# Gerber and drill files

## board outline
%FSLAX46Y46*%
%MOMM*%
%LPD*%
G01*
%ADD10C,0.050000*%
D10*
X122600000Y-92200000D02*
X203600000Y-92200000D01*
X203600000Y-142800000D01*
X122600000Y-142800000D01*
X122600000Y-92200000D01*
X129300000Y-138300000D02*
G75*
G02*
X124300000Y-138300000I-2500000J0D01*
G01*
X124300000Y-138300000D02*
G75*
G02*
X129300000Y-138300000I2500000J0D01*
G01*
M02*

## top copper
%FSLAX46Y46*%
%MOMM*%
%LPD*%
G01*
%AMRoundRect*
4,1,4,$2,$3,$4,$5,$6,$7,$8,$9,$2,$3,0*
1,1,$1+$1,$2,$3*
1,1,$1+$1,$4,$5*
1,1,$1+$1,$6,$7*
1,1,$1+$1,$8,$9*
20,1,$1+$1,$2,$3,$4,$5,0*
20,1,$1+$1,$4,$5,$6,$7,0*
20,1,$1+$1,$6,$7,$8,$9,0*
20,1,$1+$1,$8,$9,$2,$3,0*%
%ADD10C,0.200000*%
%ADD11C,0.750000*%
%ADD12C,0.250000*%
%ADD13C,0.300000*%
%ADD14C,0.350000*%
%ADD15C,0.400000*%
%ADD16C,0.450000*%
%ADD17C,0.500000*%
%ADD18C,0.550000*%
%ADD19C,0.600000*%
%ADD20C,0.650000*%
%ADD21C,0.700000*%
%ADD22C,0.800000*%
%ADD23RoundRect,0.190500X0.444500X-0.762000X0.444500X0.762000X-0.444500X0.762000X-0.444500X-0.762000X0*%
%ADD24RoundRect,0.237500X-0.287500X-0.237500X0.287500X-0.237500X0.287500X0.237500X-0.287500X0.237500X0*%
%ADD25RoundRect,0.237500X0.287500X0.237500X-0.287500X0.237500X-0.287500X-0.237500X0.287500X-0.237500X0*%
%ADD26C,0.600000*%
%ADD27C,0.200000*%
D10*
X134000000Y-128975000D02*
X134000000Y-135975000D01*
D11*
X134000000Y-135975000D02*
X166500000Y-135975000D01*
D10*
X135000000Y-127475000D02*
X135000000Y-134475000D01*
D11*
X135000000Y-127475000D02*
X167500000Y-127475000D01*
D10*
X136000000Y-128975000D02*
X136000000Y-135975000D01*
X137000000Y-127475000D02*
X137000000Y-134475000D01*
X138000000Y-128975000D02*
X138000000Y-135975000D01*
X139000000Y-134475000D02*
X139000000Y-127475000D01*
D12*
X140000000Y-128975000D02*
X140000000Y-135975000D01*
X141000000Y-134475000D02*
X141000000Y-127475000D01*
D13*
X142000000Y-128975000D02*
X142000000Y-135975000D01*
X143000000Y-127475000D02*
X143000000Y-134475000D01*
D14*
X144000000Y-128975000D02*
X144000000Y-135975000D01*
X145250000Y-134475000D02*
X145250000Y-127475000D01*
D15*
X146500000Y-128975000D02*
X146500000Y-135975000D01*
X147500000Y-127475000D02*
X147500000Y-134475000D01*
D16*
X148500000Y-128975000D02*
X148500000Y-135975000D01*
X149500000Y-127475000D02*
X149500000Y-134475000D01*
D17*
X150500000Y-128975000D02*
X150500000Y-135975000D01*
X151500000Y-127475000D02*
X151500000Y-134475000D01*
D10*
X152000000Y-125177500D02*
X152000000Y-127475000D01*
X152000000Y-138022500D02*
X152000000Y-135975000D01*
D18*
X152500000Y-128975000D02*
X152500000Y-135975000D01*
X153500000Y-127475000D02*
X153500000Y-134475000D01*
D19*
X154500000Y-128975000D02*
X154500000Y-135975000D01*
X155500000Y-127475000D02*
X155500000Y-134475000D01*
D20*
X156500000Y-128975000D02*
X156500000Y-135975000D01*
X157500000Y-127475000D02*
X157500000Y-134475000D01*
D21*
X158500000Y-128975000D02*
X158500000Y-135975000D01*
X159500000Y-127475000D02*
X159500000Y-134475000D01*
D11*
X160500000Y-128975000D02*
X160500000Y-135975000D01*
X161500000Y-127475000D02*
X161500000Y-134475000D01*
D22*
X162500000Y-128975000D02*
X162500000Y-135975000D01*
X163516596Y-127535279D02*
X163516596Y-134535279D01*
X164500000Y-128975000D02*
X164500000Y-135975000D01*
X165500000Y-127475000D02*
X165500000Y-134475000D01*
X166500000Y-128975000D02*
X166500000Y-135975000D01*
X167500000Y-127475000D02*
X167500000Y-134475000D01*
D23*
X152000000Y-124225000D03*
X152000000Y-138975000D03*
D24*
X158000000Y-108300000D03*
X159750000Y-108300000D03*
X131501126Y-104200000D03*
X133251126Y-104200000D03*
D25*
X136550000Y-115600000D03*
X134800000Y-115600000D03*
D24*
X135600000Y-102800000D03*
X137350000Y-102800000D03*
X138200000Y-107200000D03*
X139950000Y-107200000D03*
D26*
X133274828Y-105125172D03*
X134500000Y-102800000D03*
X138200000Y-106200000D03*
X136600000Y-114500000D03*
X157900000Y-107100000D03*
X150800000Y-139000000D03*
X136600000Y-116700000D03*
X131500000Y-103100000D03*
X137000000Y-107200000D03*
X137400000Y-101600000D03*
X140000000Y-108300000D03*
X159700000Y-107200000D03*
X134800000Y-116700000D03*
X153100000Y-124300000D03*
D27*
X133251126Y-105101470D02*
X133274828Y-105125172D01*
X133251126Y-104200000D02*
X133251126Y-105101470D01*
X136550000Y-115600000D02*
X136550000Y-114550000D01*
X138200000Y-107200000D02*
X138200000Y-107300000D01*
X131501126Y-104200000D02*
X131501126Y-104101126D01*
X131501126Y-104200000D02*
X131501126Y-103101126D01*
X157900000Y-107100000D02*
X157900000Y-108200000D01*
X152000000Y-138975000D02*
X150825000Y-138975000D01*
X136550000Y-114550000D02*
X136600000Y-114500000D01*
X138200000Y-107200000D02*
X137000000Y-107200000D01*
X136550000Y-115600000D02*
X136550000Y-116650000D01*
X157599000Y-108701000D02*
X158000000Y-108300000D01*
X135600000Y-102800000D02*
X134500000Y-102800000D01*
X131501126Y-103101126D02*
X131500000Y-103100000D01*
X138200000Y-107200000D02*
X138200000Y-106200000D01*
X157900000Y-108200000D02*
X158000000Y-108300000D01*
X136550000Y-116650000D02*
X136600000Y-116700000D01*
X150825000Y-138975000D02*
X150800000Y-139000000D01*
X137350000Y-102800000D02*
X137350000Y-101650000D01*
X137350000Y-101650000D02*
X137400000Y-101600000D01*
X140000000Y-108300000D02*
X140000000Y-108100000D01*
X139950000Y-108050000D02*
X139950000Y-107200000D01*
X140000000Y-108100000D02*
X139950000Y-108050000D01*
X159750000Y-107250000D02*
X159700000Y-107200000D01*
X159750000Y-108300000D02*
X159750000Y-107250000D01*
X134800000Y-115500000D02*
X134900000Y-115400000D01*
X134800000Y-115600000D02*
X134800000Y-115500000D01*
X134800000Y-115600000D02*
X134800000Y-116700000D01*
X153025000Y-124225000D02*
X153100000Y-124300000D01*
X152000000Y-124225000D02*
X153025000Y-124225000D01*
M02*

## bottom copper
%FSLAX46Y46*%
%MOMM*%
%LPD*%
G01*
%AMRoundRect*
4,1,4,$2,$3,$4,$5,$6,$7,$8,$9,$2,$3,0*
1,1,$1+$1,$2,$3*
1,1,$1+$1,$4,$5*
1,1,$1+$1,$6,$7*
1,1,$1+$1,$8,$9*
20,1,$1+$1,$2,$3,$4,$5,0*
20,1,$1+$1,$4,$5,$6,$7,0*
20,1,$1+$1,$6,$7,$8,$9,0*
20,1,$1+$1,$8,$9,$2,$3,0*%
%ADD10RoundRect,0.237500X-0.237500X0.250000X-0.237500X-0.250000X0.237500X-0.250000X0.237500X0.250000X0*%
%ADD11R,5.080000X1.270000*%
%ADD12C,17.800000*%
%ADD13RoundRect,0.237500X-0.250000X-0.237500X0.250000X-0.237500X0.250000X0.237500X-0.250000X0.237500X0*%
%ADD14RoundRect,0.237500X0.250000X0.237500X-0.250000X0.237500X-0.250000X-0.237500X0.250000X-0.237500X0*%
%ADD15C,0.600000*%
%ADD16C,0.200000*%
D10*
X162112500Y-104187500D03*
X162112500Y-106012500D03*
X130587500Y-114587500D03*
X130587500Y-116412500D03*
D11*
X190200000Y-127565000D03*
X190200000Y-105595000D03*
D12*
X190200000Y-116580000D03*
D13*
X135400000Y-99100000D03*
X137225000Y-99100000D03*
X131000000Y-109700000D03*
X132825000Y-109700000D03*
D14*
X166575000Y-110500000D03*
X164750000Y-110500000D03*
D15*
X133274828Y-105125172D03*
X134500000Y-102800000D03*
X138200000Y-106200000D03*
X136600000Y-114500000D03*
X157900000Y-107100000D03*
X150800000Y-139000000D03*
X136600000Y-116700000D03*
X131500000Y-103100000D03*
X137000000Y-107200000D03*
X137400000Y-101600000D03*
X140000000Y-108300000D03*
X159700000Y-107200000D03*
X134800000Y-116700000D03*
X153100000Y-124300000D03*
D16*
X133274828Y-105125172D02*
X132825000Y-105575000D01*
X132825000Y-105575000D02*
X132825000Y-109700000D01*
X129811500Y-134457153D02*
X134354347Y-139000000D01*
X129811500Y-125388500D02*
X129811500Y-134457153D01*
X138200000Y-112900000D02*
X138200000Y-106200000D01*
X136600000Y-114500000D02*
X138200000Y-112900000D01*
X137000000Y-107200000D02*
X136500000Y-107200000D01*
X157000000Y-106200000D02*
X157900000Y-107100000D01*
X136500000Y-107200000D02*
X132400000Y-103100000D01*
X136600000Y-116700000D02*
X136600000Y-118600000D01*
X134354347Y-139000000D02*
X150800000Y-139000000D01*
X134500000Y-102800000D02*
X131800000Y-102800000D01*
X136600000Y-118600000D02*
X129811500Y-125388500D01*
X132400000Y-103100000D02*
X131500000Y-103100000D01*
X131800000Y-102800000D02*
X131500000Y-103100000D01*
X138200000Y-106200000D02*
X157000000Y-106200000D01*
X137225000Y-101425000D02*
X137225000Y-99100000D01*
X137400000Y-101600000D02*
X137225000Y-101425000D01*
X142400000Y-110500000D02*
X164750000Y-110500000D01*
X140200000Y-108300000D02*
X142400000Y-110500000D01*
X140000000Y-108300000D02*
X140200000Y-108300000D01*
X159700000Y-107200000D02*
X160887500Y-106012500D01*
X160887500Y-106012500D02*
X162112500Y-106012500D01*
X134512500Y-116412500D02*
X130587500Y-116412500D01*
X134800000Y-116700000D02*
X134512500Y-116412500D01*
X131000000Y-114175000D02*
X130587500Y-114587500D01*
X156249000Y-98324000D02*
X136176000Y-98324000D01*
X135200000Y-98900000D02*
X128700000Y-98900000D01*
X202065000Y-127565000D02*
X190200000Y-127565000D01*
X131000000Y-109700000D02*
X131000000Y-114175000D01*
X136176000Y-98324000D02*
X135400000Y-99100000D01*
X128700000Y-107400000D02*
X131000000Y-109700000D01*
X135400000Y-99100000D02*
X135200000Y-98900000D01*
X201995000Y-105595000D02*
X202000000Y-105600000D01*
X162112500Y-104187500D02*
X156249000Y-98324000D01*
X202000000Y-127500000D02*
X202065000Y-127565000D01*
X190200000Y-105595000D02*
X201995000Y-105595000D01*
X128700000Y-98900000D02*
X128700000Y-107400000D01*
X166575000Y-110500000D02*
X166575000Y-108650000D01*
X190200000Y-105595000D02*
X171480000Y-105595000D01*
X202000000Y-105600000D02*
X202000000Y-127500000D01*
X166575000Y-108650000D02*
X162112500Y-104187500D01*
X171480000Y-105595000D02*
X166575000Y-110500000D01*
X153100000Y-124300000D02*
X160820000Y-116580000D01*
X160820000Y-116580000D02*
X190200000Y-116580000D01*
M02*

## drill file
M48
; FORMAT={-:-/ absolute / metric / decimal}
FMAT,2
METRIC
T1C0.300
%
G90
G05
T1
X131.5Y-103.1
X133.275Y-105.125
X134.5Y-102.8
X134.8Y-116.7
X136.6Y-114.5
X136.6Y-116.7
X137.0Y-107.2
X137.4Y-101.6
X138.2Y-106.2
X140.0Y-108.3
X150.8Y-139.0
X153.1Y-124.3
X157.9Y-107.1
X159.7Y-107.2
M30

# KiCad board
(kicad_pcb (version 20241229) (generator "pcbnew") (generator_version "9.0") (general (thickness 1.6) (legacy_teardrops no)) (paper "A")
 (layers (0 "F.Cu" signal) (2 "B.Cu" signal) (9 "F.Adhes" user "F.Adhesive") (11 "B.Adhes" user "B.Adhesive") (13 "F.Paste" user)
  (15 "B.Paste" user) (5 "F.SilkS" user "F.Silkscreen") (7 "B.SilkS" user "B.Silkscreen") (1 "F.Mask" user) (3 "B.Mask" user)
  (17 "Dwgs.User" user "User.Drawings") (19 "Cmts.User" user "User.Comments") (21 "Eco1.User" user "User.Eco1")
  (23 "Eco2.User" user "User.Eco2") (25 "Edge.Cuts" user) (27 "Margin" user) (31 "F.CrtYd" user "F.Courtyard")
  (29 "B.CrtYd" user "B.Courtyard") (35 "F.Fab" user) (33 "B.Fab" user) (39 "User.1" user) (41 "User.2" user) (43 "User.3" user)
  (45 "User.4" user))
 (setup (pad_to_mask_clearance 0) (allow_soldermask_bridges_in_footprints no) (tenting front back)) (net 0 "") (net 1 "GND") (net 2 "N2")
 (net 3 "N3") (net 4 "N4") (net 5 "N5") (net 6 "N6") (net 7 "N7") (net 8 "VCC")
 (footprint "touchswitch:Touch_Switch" (layer "F.Cu") (at 152 131.475 90)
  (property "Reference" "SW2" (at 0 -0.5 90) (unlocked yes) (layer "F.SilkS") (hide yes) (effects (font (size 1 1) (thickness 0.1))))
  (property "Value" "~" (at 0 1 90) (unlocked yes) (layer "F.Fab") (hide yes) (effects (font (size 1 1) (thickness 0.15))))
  (fp_line (start 2.5 -18) (end -4.5 -18) (stroke (width 0.2) (type default)) (layer "F.Cu"))
  (fp_line (start -4.5 -18) (end -4.5 14.5) (stroke (width 0.75) (type default)) (layer "F.Cu"))
  (fp_line (start 4 -17) (end -3 -17) (stroke (width 0.2) (type default)) (layer "F.Cu"))
  (fp_line (start 4 -17) (end 4 15.5) (stroke (width 0.75) (type default)) (layer "F.Cu"))
  (fp_line (start 2.5 -16) (end -4.5 -16) (stroke (width 0.2) (type default)) (layer "F.Cu"))
  (fp_line (start 4 -15) (end -3 -15) (stroke (width 0.2) (type default)) (layer "F.Cu"))
  (fp_line (start 2.5 -14) (end -4.5 -14) (stroke (width 0.2) (type default)) (layer "F.Cu"))
  (fp_line (start -3 -13) (end 4 -13) (stroke (width 0.2) (type default)) (layer "F.Cu"))
  (fp_line (start 2.5 -12) (end -4.5 -12) (stroke (width 0.25) (type default)) (layer "F.Cu"))
  (fp_line (start -3 -11) (end 4 -11) (stroke (width 0.25) (type default)) (layer "F.Cu"))
  (fp_line (start 2.5 -10) (end -4.5 -10) (stroke (width 0.3) (type default)) (layer "F.Cu"))
  (fp_line (start 4 -9) (end -3 -9) (stroke (width 0.3) (type default)) (layer "F.Cu"))
  (fp_line (start 2.5 -8) (end -4.5 -8) (stroke (width 0.35) (type default)) (layer "F.Cu"))
  (fp_line (start -3 -6.75) (end 4 -6.75) (stroke (width 0.35) (type default)) (layer "F.Cu"))
  (fp_line (start 2.5 -5.5) (end -4.5 -5.5) (stroke (width 0.4) (type default)) (layer "F.Cu"))
  (fp_line (start 4 -4.5) (end -3 -4.5) (stroke (width 0.4) (type default)) (layer "F.Cu"))
  (fp_line (start 2.5 -3.5) (end -4.5 -3.5) (stroke (width 0.45) (type default)) (layer "F.Cu"))
  (fp_line (start 4 -2.5) (end -3 -2.5) (stroke (width 0.45) (type default)) (layer "F.Cu"))
  (fp_line (start 2.5 -1.5) (end -4.5 -1.5) (stroke (width 0.5) (type default)) (layer "F.Cu"))
  (fp_line (start 4 -0.5) (end -3 -0.5) (stroke (width 0.5) (type default)) (layer "F.Cu"))
  (fp_line (start 6.2975 0) (end 4 0) (stroke (width 0.2) (type default)) (layer "F.Cu"))
  (fp_line (start -6.5475 0) (end -4.5 0) (stroke (width 0.2) (type default)) (layer "F.Cu"))
  (fp_line (start 2.5 0.5) (end -4.5 0.5) (stroke (width 0.55) (type default)) (layer "F.Cu"))
  (fp_line (start 4 1.5) (end -3 1.5) (stroke (width 0.55) (type default)) (layer "F.Cu"))
  (fp_line (start 2.5 2.5) (end -4.5 2.5) (stroke (width 0.6) (type default)) (layer "F.Cu"))
  (fp_line (start 4 3.5) (end -3 3.5) (stroke (width 0.6) (type default)) (layer "F.Cu"))
  (fp_line (start 2.5 4.5) (end -4.5 4.5) (stroke (width 0.65) (type default)) (layer "F.Cu"))
  (fp_line (start 4 5.5) (end -3 5.5) (stroke (width 0.65) (type default)) (layer "F.Cu"))
  (fp_line (start 2.5 6.5) (end -4.5 6.5) (stroke (width 0.7) (type default)) (layer "F.Cu"))
  (fp_line (start 4 7.5) (end -3 7.5) (stroke (width 0.7) (type default)) (layer "F.Cu"))
  (fp_line (start 2.5 8.5) (end -4.5 8.5) (stroke (width 0.75) (type default)) (layer "F.Cu"))
  (fp_line (start 4 9.5) (end -3 9.5) (stroke (width 0.75) (type default)) (layer "F.Cu"))
  (fp_line (start 2.5 10.5) (end -4.5 10.5) (stroke (width 0.8) (type default)) (layer "F.Cu"))
  (fp_line (start 3.939721 11.516596) (end -3.060279 11.516596) (stroke (width 0.8) (type default)) (layer "F.Cu"))
  (fp_line (start 2.5 12.5) (end -4.5 12.5) (stroke (width 0.8) (type default)) (layer "F.Cu"))
  (fp_line (start 4 13.5) (end -3 13.5) (stroke (width 0.8) (type default)) (layer "F.Cu"))
  (fp_line (start 2.5 14.5) (end -4.5 14.5) (stroke (width 0.8) (type default)) (layer "F.Cu"))
  (fp_line (start 4 15.5) (end -3 15.5) (stroke (width 0.8) (type default)) (layer "F.Cu"))
  (pad "1" smd roundrect (at 7.25 0 90) (size 1.905 1.27) (layers "F.Cu" "F.Mask" "F.Paste") (roundrect_rratio 0.15) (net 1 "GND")
   (thermal_bridge_angle 45))
  (pad "2" smd roundrect (at -7.5 0 90) (size 1.905 1.27) (layers "F.Cu" "F.Mask" "F.Paste") (roundrect_rratio 0.15) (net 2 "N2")
   (thermal_bridge_angle 45)))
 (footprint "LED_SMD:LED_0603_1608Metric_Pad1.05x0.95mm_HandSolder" (layer "F.Cu") (at 158.875 108.3)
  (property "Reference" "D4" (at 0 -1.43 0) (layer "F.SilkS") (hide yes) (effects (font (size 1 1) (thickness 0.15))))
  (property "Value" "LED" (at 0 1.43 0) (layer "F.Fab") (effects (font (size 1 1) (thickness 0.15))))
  (pad "1" smd roundrect (at -0.875 0) (size 1.05 0.95) (layers "F.Cu" "F.Mask" "F.Paste") (roundrect_rratio 0.25) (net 2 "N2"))
  (pad "2" smd roundrect (at 0.875 0) (size 1.05 0.95) (layers "F.Cu" "F.Mask" "F.Paste") (roundrect_rratio 0.25) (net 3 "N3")))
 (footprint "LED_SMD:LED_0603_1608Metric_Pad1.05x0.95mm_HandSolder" (layer "F.Cu") (at 132.376126 104.2)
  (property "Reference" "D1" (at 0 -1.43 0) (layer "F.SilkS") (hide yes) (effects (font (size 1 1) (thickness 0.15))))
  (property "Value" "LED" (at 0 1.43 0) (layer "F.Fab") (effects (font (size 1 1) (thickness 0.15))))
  (pad "1" smd roundrect (at -0.875 0) (size 1.05 0.95) (layers "F.Cu" "F.Mask" "F.Paste") (roundrect_rratio 0.25) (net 2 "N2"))
  (pad "2" smd roundrect (at 0.875 0) (size 1.05 0.95) (layers "F.Cu" "F.Mask" "F.Paste") (roundrect_rratio 0.25) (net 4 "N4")))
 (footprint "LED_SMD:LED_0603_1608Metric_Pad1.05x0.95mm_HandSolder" (layer "F.Cu") (at 135.675 115.6 180)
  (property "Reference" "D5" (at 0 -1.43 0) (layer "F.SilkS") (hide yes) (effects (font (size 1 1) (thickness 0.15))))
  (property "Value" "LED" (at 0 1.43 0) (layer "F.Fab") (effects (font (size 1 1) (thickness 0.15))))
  (pad "1" smd roundrect (at -0.875 0 180) (size 1.05 0.95) (layers "F.Cu" "F.Mask" "F.Paste") (roundrect_rratio 0.25) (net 2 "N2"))
  (pad "2" smd roundrect (at 0.875 0 180) (size 1.05 0.95) (layers "F.Cu" "F.Mask" "F.Paste") (roundrect_rratio 0.25) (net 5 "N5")))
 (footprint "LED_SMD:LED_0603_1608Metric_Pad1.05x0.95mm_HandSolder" (layer "F.Cu") (at 136.475 102.8)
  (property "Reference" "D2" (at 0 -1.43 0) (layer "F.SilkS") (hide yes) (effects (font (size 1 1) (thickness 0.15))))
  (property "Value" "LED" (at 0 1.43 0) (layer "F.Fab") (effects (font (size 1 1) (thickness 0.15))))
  (pad "1" smd roundrect (at -0.875 0) (size 1.05 0.95) (layers "F.Cu" "F.Mask" "F.Paste") (roundrect_rratio 0.25) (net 2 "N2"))
  (pad "2" smd roundrect (at 0.875 0) (size 1.05 0.95) (layers "F.Cu" "F.Mask" "F.Paste") (roundrect_rratio 0.25) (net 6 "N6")))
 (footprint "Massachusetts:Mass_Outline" (layer "F.Cu") (at 321.080166 206.806759)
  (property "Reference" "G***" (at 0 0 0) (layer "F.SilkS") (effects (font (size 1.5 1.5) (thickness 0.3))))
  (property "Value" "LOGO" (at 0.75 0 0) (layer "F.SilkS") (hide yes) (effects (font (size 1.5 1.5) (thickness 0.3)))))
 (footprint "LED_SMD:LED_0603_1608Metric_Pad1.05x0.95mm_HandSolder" (layer "F.Cu") (at 139.075 107.2)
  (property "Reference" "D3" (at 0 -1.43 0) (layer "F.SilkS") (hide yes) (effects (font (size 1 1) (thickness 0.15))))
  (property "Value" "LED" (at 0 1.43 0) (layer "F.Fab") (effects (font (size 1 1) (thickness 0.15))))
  (pad "1" smd roundrect (at -0.875 0) (size 1.05 0.95) (layers "F.Cu" "F.Mask" "F.Paste") (roundrect_rratio 0.25) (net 2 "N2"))
  (pad "2" smd roundrect (at 0.875 0) (size 1.05 0.95) (layers "F.Cu" "F.Mask" "F.Paste") (roundrect_rratio 0.25) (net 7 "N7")))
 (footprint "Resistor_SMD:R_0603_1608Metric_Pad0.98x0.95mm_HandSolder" (layer "B.Cu") (at 162.1125 105.1 -90)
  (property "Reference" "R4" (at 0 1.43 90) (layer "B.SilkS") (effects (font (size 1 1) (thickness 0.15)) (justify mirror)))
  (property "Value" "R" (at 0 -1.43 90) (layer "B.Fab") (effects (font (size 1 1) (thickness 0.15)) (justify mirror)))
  (pad "1" smd roundrect (at -0.9125 0 270) (size 0.975 0.95) (layers "B.Cu" "B.Mask" "B.Paste") (roundrect_rratio 0.25) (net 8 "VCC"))
  (pad "2" smd roundrect (at 0.9125 0 270) (size 0.975 0.95) (layers "B.Cu" "B.Mask" "B.Paste") (roundrect_rratio 0.25) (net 3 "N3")))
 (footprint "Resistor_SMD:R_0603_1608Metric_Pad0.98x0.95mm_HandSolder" (layer "B.Cu") (at 130.5875 115.5 -90)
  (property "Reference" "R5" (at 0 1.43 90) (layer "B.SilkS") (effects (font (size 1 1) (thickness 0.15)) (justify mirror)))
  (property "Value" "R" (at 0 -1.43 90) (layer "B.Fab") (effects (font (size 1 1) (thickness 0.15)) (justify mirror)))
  (pad "1" smd roundrect (at -0.9125 0 270) (size 0.975 0.95) (layers "B.Cu" "B.Mask" "B.Paste") (roundrect_rratio 0.25) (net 8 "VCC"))
  (pad "2" smd roundrect (at 0.9125 0 270) (size 0.975 0.95) (layers "B.Cu" "B.Mask" "B.Paste") (roundrect_rratio 0.25) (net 5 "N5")))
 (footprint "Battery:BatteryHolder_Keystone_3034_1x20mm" (layer "B.Cu") (at 190.2 116.58 90)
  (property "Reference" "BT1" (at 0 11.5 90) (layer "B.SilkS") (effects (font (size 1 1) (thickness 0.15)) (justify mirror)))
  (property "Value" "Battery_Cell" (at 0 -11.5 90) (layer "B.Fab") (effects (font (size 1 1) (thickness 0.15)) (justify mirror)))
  (pad "1" smd rect (at -10.985 0 90) (size 1.27 5.08) (layers "B.Cu" "B.Mask" "B.Paste") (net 8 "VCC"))
  (pad "1" smd rect (at 10.985 0 90) (size 1.27 5.08) (layers "B.Cu" "B.Mask" "B.Paste") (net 8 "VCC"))
  (pad "2" smd circle (at 0 0 90) (size 17.8 17.8) (layers "B.Cu" "B.Mask") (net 1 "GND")))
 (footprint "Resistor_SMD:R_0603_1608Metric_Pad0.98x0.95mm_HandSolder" (layer "B.Cu") (at 136.3125 99.1)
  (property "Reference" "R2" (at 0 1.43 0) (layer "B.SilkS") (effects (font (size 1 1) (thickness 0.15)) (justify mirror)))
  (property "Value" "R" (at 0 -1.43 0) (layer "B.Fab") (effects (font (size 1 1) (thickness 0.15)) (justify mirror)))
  (pad "1" smd roundrect (at -0.9125 0) (size 0.975 0.95) (layers "B.Cu" "B.Mask" "B.Paste") (roundrect_rratio 0.25) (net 8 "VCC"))
  (pad "2" smd roundrect (at 0.9125 0) (size 0.975 0.95) (layers "B.Cu" "B.Mask" "B.Paste") (roundrect_rratio 0.25) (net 6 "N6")))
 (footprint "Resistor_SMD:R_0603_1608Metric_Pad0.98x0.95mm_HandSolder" (layer "B.Cu") (at 131.9125 109.7)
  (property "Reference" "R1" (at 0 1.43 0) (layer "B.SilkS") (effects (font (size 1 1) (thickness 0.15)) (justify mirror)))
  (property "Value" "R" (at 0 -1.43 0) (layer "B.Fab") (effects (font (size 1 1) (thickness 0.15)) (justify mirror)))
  (pad "1" smd roundrect (at -0.9125 0) (size 0.975 0.95) (layers "B.Cu" "B.Mask" "B.Paste") (roundrect_rratio 0.25) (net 8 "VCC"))
  (pad "2" smd roundrect (at 0.9125 0) (size 0.975 0.95) (layers "B.Cu" "B.Mask" "B.Paste") (roundrect_rratio 0.25) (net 4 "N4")))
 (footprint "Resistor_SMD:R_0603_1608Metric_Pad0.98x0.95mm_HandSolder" (layer "B.Cu") (at 165.6625 110.5 180)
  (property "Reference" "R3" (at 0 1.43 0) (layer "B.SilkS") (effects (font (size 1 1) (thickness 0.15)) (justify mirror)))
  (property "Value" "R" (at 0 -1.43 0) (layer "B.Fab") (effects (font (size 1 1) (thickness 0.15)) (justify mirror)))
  (pad "1" smd roundrect (at -0.9125 0 180) (size 0.975 0.95) (layers "B.Cu" "B.Mask" "B.Paste") (roundrect_rratio 0.25) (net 8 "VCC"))
  (pad "2" smd roundrect (at 0.9125 0 180) (size 0.975 0.95) (layers "B.Cu" "B.Mask" "B.Paste") (roundrect_rratio 0.25) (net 7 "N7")))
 (gr_rect (start 122.6 92.2) (end 203.6 142.8) (stroke (width 0.05) (type default)) (fill no) (layer "Edge.Cuts"))
 (gr_circle (center 126.8 138.3) (end 129.3 138.3) (stroke (width 0.05) (type solid)) (fill no) (layer "Edge.Cuts"))
 (segment (start 133.251126 105.10147) (end 133.274828 105.125172) (width 0.2) (layer "F.Cu") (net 4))
 (segment (start 133.251126 104.2) (end 133.251126 105.10147) (width 0.2) (layer "F.Cu") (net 4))
 (via (at 133.274828 105.125172) (size 0.6) (drill 0.3) (layers "F.Cu" "B.Cu") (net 4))
 (segment (start 133.274828 105.125172) (end 132.825 105.575) (width 0.2) (layer "B.Cu") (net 4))
 (segment (start 132.825 105.575) (end 132.825 109.7) (width 0.2) (layer "B.Cu") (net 4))
 (segment (start 136.55 115.6) (end 136.55 114.55) (width 0.2) (layer "F.Cu") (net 2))
 (segment (start 138.2 107.2) (end 138.2 107.3) (width 0.2) (layer "F.Cu") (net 2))
 (segment (start 131.501126 104.2) (end 131.501126 104.101126) (width 0.2) (layer "F.Cu") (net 2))
 (segment (start 131.501126 104.2) (end 131.501126 103.101126) (width 0.2) (layer "F.Cu") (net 2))
 (segment (start 157.9 107.1) (end 157.9 108.2) (width 0.2) (layer "F.Cu") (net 2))
 (segment (start 152 138.975) (end 150.825 138.975) (width 0.2) (layer "F.Cu") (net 2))
 (segment (start 136.55 114.55) (end 136.6 114.5) (width 0.2) (layer "F.Cu") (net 2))
 (segment (start 138.2 107.2) (end 137 107.2) (width 0.2) (layer "F.Cu") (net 2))
 (segment (start 136.55 115.6) (end 136.55 116.65) (width 0.2) (layer "F.Cu") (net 2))
 (segment (start 157.599 108.701) (end 158 108.3) (width 0.2) (layer "F.Cu") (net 2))
 (segment (start 135.6 102.8) (end 134.5 102.8) (width 0.2) (layer "F.Cu") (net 2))
 (segment (start 131.501126 103.101126) (end 131.5 103.1) (width 0.2) (layer "F.Cu") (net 2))
 (segment (start 138.2 107.2) (end 138.2 106.2) (width 0.2) (layer "F.Cu") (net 2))
 (segment (start 157.9 108.2) (end 158 108.3) (width 0.2) (layer "F.Cu") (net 2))
 (segment (start 136.55 116.65) (end 136.6 116.7) (width 0.2) (layer "F.Cu") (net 2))
 (segment (start 150.825 138.975) (end 150.8 139) (width 0.2) (layer "F.Cu") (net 2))
 (via (at 134.5 102.8) (size 0.6) (drill 0.3) (layers "F.Cu" "B.Cu") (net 2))
 (via (at 138.2 106.2) (size 0.6) (drill 0.3) (layers "F.Cu" "B.Cu") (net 2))
 (via (at 136.6 114.5) (size 0.6) (drill 0.3) (layers "F.Cu" "B.Cu") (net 2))
 (via (at 157.9 107.1) (size 0.6) (drill 0.3) (layers "F.Cu" "B.Cu") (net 2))
 (via (at 150.8 139) (size 0.6) (drill 0.3) (layers "F.Cu" "B.Cu") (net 2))
 (via (at 136.6 116.7) (size 0.6) (drill 0.3) (layers "F.Cu" "B.Cu") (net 2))
 (via (at 131.5 103.1) (size 0.6) (drill 0.3) (layers "F.Cu" "B.Cu") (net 2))
 (via (at 137 107.2) (size 0.6) (drill 0.3) (layers "F.Cu" "B.Cu") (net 2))
 (segment (start 129.8115 134.457153) (end 134.354347 139) (width 0.2) (layer "B.Cu") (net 2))
 (segment (start 129.8115 125.3885) (end 129.8115 134.457153) (width 0.2) (layer "B.Cu") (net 2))
 (segment (start 138.2 112.9) (end 138.2 106.2) (width 0.2) (layer "B.Cu") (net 2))
 (segment (start 136.6 114.5) (end 138.2 112.9) (width 0.2) (layer "B.Cu") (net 2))
 (segment (start 137 107.2) (end 136.5 107.2) (width 0.2) (layer "B.Cu") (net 2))
 (segment (start 157 106.2) (end 157.9 107.1) (width 0.2) (layer "B.Cu") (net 2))
 (segment (start 136.5 107.2) (end 132.4 103.1) (width 0.2) (layer "B.Cu") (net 2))
 (segment (start 136.6 116.7) (end 136.6 118.6) (width 0.2) (layer "B.Cu") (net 2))
 (segment (start 134.354347 139) (end 150.8 139) (width 0.2) (layer "B.Cu") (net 2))
 (segment (start 134.5 102.8) (end 131.8 102.8) (width 0.2) (layer "B.Cu") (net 2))
 (segment (start 136.6 118.6) (end 129.8115 125.3885) (width 0.2) (layer "B.Cu") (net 2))
 (segment (start 132.4 103.1) (end 131.5 103.1) (width 0.2) (layer "B.Cu") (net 2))
 (segment (start 131.8 102.8) (end 131.5 103.1) (width 0.2) (layer "B.Cu") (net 2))
 (segment (start 138.2 106.2) (end 157 106.2) (width 0.2) (layer "B.Cu") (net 2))
 (segment (start 137.35 102.8) (end 137.35 101.65) (width 0.2) (layer "F.Cu") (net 6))
 (segment (start 137.35 101.65) (end 137.4 101.6) (width 0.2) (layer "F.Cu") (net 6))
 (via (at 137.4 101.6) (size 0.6) (drill 0.3) (layers "F.Cu" "B.Cu") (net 6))
 (segment (start 137.225 101.425) (end 137.225 99.1) (width 0.2) (layer "B.Cu") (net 6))
 (segment (start 137.4 101.6) (end 137.225 101.425) (width 0.2) (layer "B.Cu") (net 6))
 (segment (start 140 108.3) (end 140 108.1) (width 0.2) (layer "F.Cu") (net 7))
 (segment (start 139.95 108.05) (end 139.95 107.2) (width 0.2) (layer "F.Cu") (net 7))
 (segment (start 140 108.1) (end 139.95 108.05) (width 0.2) (layer "F.Cu") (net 7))
 (via (at 140 108.3) (size 0.6) (drill 0.3) (layers "F.Cu" "B.Cu") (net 7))
 (segment (start 142.4 110.5) (end 164.75 110.5) (width 0.2) (layer "B.Cu") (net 7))
 (segment (start 140.2 108.3) (end 142.4 110.5) (width 0.2) (layer "B.Cu") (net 7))
 (segment (start 140 108.3) (end 140.2 108.3) (width 0.2) (layer "B.Cu") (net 7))
 (segment (start 159.75 107.25) (end 159.7 107.2) (width 0.2) (layer "F.Cu") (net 3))
 (segment (start 159.75 108.3) (end 159.75 107.25) (width 0.2) (layer "F.Cu") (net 3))
 (via (at 159.7 107.2) (size 0.6) (drill 0.3) (layers "F.Cu" "B.Cu") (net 3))
 (segment (start 159.7 107.2) (end 160.8875 106.0125) (width 0.2) (layer "B.Cu") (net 3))
 (segment (start 160.8875 106.0125) (end 162.1125 106.0125) (width 0.2) (layer "B.Cu") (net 3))
 (segment (start 134.8 115.5) (end 134.9 115.4) (width 0.2) (layer "F.Cu") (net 5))
 (segment (start 134.8 115.6) (end 134.8 115.5) (width 0.2) (layer "F.Cu") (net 5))
 (segment (start 134.8 115.6) (end 134.8 116.7) (width 0.2) (layer "F.Cu") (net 5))
 (via (at 134.8 116.7) (size 0.6) (drill 0.3) (layers "F.Cu" "B.Cu") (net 5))
 (segment (start 134.5125 116.4125) (end 130.5875 116.4125) (width 0.2) (layer "B.Cu") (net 5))
 (segment (start 134.8 116.7) (end 134.5125 116.4125) (width 0.2) (layer "B.Cu") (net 5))
 (segment (start 131 114.175) (end 130.5875 114.5875) (width 0.2) (layer "B.Cu") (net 8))
 (segment (start 156.249 98.324) (end 136.176 98.324) (width 0.2) (layer "B.Cu") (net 8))
 (segment (start 135.2 98.9) (end 128.7 98.9) (width 0.2) (layer "B.Cu") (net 8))
 (segment (start 202.065 127.565) (end 190.2 127.565) (width 0.2) (layer "B.Cu") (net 8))
 (segment (start 131 109.7) (end 131 114.175) (width 0.2) (layer "B.Cu") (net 8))
 (segment (start 136.176 98.324) (end 135.4 99.1) (width 0.2) (layer "B.Cu") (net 8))
 (segment (start 128.7 107.4) (end 131 109.7) (width 0.2) (layer "B.Cu") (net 8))
 (segment (start 135.4 99.1) (end 135.2 98.9) (width 0.2) (layer "B.Cu") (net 8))
 (segment (start 201.995 105.595) (end 202 105.6) (width 0.2) (layer "B.Cu") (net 8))
 (segment (start 162.1125 104.1875) (end 156.249 98.324) (width 0.2) (layer "B.Cu") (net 8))
 (segment (start 202 127.5) (end 202.065 127.565) (width 0.2) (layer "B.Cu") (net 8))
 (segment (start 190.2 105.595) (end 201.995 105.595) (width 0.2) (layer "B.Cu") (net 8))
 (segment (start 128.7 98.9) (end 128.7 107.4) (width 0.2) (layer "B.Cu") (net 8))
 (segment (start 166.575 110.5) (end 166.575 108.65) (width 0.2) (layer "B.Cu") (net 8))
 (segment (start 190.2 105.595) (end 171.48 105.595) (width 0.2) (layer "B.Cu") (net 8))
 (segment (start 202 105.6) (end 202 127.5) (width 0.2) (layer "B.Cu") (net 8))
 (segment (start 166.575 108.65) (end 162.1125 104.1875) (width 0.2) (layer "B.Cu") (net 8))
 (segment (start 171.48 105.595) (end 166.575 110.5) (width 0.2) (layer "B.Cu") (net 8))
 (segment (start 153.025 124.225) (end 153.1 124.3) (width 0.2) (layer "F.Cu") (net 1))
 (segment (start 152 124.225) (end 153.025 124.225) (width 0.2) (layer "F.Cu") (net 1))
 (via (at 153.1 124.3) (size 0.6) (drill 0.3) (layers "F.Cu" "B.Cu") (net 1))
 (segment (start 153.1 124.3) (end 160.82 116.58) (width 0.2) (layer "B.Cu") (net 1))
 (segment (start 160.82 116.58) (end 190.2 116.58) (width 0.2) (layer "B.Cu") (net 1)))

